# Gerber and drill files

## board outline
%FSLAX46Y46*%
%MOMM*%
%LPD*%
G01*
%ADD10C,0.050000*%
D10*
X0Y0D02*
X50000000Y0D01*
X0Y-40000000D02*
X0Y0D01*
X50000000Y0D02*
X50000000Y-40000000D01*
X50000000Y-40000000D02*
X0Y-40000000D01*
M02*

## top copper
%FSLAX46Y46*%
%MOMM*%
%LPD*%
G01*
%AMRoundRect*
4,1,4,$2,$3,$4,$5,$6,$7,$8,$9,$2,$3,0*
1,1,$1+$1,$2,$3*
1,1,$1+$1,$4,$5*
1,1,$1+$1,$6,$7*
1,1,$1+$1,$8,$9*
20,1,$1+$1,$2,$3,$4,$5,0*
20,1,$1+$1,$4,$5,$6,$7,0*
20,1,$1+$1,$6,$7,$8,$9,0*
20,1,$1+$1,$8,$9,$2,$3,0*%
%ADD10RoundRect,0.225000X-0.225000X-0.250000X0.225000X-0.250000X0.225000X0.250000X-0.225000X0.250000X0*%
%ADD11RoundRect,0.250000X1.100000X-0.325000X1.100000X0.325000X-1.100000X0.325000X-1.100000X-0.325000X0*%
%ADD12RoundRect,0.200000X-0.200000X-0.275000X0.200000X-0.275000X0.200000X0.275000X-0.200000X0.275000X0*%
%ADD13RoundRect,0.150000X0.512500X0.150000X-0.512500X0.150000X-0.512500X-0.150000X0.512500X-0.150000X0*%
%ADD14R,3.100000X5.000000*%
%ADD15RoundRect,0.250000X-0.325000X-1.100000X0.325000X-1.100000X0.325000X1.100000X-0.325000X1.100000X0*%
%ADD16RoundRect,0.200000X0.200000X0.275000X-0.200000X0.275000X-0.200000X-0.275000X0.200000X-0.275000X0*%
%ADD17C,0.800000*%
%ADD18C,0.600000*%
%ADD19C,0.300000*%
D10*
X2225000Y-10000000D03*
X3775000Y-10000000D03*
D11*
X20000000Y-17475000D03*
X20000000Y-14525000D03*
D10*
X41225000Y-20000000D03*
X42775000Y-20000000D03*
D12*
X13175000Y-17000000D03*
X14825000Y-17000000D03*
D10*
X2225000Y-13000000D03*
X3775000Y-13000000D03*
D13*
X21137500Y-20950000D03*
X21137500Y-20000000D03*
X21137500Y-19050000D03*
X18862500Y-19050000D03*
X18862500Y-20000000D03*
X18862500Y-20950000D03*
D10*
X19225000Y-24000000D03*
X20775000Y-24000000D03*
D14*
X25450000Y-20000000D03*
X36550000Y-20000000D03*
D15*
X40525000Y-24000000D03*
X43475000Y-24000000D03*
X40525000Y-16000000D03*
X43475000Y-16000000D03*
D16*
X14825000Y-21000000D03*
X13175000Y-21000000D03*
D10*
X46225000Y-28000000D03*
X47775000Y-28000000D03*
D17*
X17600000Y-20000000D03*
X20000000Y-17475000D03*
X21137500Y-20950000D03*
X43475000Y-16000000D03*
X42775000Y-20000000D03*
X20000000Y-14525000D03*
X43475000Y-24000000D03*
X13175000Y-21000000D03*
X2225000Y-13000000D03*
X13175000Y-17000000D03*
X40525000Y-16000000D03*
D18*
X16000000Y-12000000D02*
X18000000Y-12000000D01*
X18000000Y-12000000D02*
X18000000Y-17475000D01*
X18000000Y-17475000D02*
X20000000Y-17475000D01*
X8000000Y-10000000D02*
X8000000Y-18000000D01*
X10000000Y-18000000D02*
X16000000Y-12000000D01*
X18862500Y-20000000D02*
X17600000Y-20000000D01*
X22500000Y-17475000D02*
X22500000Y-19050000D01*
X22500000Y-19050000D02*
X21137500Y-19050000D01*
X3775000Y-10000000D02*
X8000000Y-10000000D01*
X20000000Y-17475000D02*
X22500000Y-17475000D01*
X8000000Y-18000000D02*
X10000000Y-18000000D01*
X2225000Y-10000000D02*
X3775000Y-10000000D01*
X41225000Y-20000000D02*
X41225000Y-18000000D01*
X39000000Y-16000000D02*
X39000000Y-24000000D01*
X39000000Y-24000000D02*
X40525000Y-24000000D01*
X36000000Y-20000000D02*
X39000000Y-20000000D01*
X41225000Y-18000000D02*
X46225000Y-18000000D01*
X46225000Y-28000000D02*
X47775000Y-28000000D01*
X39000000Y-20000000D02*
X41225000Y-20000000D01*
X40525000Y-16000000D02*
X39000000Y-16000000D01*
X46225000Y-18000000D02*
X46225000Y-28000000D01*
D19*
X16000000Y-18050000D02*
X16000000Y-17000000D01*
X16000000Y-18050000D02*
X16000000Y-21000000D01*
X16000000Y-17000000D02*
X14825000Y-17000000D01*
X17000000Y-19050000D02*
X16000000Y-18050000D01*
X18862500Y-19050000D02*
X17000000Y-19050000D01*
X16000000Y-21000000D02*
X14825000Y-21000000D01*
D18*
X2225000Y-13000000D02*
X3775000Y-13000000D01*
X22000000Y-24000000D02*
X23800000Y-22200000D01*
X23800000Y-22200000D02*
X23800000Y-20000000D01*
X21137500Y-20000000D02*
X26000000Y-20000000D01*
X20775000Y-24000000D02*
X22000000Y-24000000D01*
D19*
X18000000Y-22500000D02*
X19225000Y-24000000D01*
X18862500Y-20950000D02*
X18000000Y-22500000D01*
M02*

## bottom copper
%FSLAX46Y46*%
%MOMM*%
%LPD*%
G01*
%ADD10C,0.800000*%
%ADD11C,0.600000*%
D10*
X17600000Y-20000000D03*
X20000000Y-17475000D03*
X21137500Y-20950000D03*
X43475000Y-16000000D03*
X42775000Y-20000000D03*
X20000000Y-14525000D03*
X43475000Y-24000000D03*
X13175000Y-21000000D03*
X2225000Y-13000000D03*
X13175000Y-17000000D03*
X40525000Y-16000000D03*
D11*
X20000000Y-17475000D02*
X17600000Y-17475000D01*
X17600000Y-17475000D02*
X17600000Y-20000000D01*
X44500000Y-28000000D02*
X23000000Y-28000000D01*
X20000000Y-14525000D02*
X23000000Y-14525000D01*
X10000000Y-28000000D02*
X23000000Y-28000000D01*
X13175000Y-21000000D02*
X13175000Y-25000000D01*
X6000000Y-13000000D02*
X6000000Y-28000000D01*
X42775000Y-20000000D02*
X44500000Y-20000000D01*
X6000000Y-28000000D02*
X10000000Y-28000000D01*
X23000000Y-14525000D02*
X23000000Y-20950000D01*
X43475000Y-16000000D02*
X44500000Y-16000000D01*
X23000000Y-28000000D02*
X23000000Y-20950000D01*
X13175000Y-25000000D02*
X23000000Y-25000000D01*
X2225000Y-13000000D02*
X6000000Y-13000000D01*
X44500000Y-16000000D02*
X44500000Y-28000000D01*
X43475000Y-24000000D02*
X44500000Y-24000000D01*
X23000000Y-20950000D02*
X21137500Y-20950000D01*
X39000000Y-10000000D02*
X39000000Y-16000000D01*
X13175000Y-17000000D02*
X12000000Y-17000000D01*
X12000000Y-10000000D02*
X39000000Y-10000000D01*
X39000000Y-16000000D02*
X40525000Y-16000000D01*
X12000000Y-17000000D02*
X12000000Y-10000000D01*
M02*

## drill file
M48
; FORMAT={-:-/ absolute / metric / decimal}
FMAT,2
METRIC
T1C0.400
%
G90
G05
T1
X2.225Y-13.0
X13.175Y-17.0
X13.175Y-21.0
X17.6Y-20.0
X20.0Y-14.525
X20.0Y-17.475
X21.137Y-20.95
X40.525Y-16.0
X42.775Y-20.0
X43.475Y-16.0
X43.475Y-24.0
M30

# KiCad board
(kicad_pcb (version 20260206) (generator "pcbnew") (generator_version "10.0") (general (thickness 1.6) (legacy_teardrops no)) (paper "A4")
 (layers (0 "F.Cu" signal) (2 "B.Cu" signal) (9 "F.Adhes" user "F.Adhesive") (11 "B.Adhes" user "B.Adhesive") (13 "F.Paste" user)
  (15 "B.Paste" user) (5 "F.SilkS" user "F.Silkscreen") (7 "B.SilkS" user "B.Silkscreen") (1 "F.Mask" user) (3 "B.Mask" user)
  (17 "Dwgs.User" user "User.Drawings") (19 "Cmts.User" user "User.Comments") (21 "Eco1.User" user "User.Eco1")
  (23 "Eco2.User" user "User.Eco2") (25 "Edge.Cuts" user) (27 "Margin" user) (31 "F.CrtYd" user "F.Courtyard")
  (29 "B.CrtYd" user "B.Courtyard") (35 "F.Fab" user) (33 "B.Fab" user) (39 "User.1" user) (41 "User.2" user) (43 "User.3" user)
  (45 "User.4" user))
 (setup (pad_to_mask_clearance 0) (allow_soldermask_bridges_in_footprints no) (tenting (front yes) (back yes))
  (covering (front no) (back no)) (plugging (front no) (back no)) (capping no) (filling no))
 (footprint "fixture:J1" (layer "F.Cu") (at 3 10)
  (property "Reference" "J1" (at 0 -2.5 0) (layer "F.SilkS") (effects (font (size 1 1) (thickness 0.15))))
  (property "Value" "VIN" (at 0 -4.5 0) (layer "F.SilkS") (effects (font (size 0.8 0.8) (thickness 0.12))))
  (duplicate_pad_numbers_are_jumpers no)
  (pad "1" smd roundrect (at -0.775 0) (size 0.9 0.95) (layers "F.Cu" "F.Mask" "F.Paste") (roundrect_rratio 0.25) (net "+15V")
   (thermal_bridge_angle 45))
  (pad "2" smd roundrect (at 0.775 0) (size 0.9 0.95) (layers "F.Cu" "F.Mask" "F.Paste") (roundrect_rratio 0.25) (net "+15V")
   (thermal_bridge_angle 45)))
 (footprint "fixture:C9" (layer "F.Cu") (at 20 16 90)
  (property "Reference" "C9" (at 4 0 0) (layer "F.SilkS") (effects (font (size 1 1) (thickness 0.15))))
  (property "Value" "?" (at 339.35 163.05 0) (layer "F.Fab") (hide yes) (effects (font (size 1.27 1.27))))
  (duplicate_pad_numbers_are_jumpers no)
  (pad "1" smd roundrect (at -1.475 0 90) (size 1.15 2.7) (layers "F.Cu" "F.Mask" "F.Paste") (roundrect_rratio 0.217391) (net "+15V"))
  (pad "2" smd roundrect (at 1.475 0 90) (size 1.15 2.7) (layers "F.Cu" "F.Mask" "F.Paste") (roundrect_rratio 0.217391) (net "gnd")))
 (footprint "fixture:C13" (layer "F.Cu") (at 42 20)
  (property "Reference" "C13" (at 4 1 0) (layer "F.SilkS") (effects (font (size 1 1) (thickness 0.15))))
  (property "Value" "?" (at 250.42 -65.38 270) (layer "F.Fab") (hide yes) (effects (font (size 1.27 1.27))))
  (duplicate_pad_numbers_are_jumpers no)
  (pad "1" smd roundrect (at -0.775 0) (size 0.9 0.95) (layers "F.Cu" "F.Mask" "F.Paste") (roundrect_rratio 0.25) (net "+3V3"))
  (pad "2" smd roundrect (at 0.775 0) (size 0.9 0.95) (layers "F.Cu" "F.Mask" "F.Paste") (roundrect_rratio 0.25) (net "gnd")))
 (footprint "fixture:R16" (layer "F.Cu") (at 14 17)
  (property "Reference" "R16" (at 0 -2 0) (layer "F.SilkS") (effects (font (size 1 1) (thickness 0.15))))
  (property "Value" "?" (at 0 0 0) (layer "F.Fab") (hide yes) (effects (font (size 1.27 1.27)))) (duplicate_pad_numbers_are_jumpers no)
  (pad "1" smd roundrect (at -0.825 0) (size 0.8 0.95) (layers "F.Cu" "F.Mask" "F.Paste") (roundrect_rratio 0.25) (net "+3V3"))
  (pad "2" smd roundrect (at 0.825 0) (size 0.8 0.95) (layers "F.Cu" "F.Mask" "F.Paste") (roundrect_rratio 0.25) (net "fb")))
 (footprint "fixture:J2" (layer "F.Cu") (at 3 13)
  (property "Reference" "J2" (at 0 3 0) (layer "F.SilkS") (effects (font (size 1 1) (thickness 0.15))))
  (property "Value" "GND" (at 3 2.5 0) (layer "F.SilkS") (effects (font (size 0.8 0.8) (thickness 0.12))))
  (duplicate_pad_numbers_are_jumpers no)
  (pad "1" smd roundrect (at -0.775 0) (size 0.9 0.95) (layers "F.Cu" "F.Mask" "F.Paste") (roundrect_rratio 0.25) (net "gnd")
   (thermal_bridge_angle 45))
  (pad "2" smd roundrect (at 0.775 0) (size 0.9 0.95) (layers "F.Cu" "F.Mask" "F.Paste") (roundrect_rratio 0.25) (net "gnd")
   (thermal_bridge_angle 45)))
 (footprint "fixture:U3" (layer "F.Cu") (at 20 20 180)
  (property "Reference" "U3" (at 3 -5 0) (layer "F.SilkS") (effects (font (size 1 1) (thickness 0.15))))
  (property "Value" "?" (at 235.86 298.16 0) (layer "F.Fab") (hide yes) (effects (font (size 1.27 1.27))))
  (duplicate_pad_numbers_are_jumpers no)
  (pad "1" smd roundrect (at -1.1375 -0.95 180) (size 1.325 0.6) (layers "F.Cu" "F.Mask" "F.Paste") (roundrect_rratio 0.25) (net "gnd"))
  (pad "2" smd roundrect (at -1.1375 0 180) (size 1.325 0.6) (layers "F.Cu" "F.Mask" "F.Paste") (roundrect_rratio 0.25) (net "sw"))
  (pad "3" smd roundrect (at -1.1375 0.95 180) (size 1.325 0.6) (layers "F.Cu" "F.Mask" "F.Paste") (roundrect_rratio 0.25) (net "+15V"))
  (pad "4" smd roundrect (at 1.1375 0.95 180) (size 1.325 0.6) (layers "F.Cu" "F.Mask" "F.Paste") (roundrect_rratio 0.25) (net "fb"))
  (pad "5" smd roundrect (at 1.1375 0 180) (size 1.325 0.6) (layers "F.Cu" "F.Mask" "F.Paste") (roundrect_rratio 0.25) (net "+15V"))
  (pad "6" smd roundrect (at 1.1375 -0.95 180) (size 1.325 0.6) (layers "F.Cu" "F.Mask" "F.Paste") (roundrect_rratio 0.25) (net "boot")))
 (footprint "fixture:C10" (layer "F.Cu") (at 20 24)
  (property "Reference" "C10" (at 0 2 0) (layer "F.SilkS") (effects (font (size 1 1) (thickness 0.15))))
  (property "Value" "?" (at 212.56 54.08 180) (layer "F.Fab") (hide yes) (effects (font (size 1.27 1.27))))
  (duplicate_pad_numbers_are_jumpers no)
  (pad "1" smd roundrect (at -0.775 0) (size 0.9 0.95) (layers "F.Cu" "F.Mask" "F.Paste") (roundrect_rratio 0.25) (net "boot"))
  (pad "2" smd roundrect (at 0.775 0) (size 0.9 0.95) (layers "F.Cu" "F.Mask" "F.Paste") (roundrect_rratio 0.25) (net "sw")))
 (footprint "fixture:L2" (layer "F.Cu") (at 31 20)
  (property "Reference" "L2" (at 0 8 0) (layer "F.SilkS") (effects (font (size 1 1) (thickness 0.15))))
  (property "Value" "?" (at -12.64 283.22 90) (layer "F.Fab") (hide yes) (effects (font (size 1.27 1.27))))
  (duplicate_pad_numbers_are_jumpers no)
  (pad "1" smd rect (at -5.55 0) (size 3.1 5) (layers "F.Cu" "F.Mask" "F.Paste") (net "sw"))
  (pad "2" smd rect (at 5.55 0) (size 3.1 5) (layers "F.Cu" "F.Mask" "F.Paste") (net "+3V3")))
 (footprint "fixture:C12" (layer "F.Cu") (at 42 24)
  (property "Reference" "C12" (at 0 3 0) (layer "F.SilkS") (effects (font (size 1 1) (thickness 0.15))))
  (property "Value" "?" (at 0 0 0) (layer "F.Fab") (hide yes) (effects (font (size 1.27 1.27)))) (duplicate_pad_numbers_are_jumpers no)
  (pad "1" smd roundrect (at -1.475 0) (size 1.15 2.7) (layers "F.Cu" "F.Mask" "F.Paste") (roundrect_rratio 0.217391) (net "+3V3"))
  (pad "2" smd roundrect (at 1.475 0) (size 1.15 2.7) (layers "F.Cu" "F.Mask" "F.Paste") (roundrect_rratio 0.217391) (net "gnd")))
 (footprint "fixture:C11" (layer "F.Cu") (at 42 16)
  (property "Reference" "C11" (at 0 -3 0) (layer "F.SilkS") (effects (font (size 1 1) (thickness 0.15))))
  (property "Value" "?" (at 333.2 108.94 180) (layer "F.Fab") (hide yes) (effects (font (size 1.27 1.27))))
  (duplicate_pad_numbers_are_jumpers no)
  (pad "1" smd roundrect (at -1.475 0) (size 1.15 2.7) (layers "F.Cu" "F.Mask" "F.Paste") (roundrect_rratio 0.217391) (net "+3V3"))
  (pad "2" smd roundrect (at 1.475 0) (size 1.15 2.7) (layers "F.Cu" "F.Mask" "F.Paste") (roundrect_rratio 0.217391) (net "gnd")))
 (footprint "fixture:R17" (layer "F.Cu") (at 14 21 180)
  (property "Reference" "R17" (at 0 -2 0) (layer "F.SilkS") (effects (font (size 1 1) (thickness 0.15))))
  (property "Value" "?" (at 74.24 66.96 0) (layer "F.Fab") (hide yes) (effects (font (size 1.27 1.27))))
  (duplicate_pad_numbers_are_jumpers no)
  (pad "1" smd roundrect (at -0.825 0 180) (size 0.8 0.95) (layers "F.Cu" "F.Mask" "F.Paste") (roundrect_rratio 0.25) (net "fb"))
  (pad "2" smd roundrect (at 0.825 0 180) (size 0.8 0.95) (layers "F.Cu" "F.Mask" "F.Paste") (roundrect_rratio 0.25) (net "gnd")))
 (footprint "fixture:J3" (layer "F.Cu") (at 47 28)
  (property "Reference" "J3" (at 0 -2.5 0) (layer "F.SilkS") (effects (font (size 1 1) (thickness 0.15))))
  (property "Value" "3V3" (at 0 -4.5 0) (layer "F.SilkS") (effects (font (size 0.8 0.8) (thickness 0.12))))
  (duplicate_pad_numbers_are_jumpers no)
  (pad "1" smd roundrect (at -0.775 0) (size 0.9 0.95) (layers "F.Cu" "F.Mask" "F.Paste") (roundrect_rratio 0.25) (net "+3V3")
   (thermal_bridge_angle 45))
  (pad "2" smd roundrect (at 0.775 0) (size 0.9 0.95) (layers "F.Cu" "F.Mask" "F.Paste") (roundrect_rratio 0.25) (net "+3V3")
   (thermal_bridge_angle 45)))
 (gr_line (start 0 0) (end 50 0) (stroke (width 0.05) (type default)) (layer "Edge.Cuts"))
 (gr_line (start 0 40) (end 0 0) (stroke (width 0.05) (type default)) (layer "Edge.Cuts"))
 (gr_line (start 50 0) (end 50 40) (stroke (width 0.05) (type default)) (layer "Edge.Cuts"))
 (gr_line (start 50 40) (end 0 40) (stroke (width 0.05) (type default)) (layer "Edge.Cuts"))
 (segment (start 16 12) (end 18 12) (width 0.6) (layer "F.Cu") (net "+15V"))
 (segment (start 18 12) (end 18 17.475) (width 0.6) (layer "F.Cu") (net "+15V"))
 (segment (start 18 17.475) (end 20 17.475) (width 0.6) (layer "F.Cu") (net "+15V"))
 (segment (start 8 10) (end 8 18) (width 0.6) (layer "F.Cu") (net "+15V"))
 (segment (start 10 18) (end 16 12) (width 0.6) (layer "F.Cu") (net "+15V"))
 (segment (start 18.8625 20) (end 17.6 20) (width 0.6) (layer "F.Cu") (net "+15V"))
 (segment (start 22.5 17.475) (end 22.5 19.05) (width 0.6) (layer "F.Cu") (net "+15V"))
 (segment (start 22.5 19.05) (end 21.1375 19.05) (width 0.6) (layer "F.Cu") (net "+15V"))
 (segment (start 3.775 10) (end 8 10) (width 0.6) (layer "F.Cu") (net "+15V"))
 (segment (start 20 17.475) (end 22.5 17.475) (width 0.6) (layer "F.Cu") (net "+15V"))
 (segment (start 8 18) (end 10 18) (width 0.6) (layer "F.Cu") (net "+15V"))
 (segment (start 2.225 10) (end 3.775 10) (width 0.6) (layer "F.Cu") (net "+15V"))
 (via (at 17.6 20) (size 0.8) (drill 0.4) (layers "F.Cu" "B.Cu") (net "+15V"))
 (via (at 20 17.475) (size 0.8) (drill 0.4) (layers "F.Cu" "B.Cu") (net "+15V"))
 (segment (start 20 17.475) (end 17.6 17.475) (width 0.6) (layer "B.Cu") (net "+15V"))
 (segment (start 17.6 17.475) (end 17.6 20) (width 0.6) (layer "B.Cu") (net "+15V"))
 (via (at 21.1375 20.95) (size 0.8) (drill 0.4) (layers "F.Cu" "B.Cu") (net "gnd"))
 (via (at 43.475 16) (size 0.8) (drill 0.4) (layers "F.Cu" "B.Cu") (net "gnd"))
 (via (at 42.775 20) (size 0.8) (drill 0.4) (layers "F.Cu" "B.Cu") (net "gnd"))
 (via (at 20 14.525) (size 0.8) (drill 0.4) (layers "F.Cu" "B.Cu") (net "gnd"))
 (via (at 43.475 24) (size 0.8) (drill 0.4) (layers "F.Cu" "B.Cu") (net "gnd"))
 (via (at 13.175 21) (size 0.8) (drill 0.4) (layers "F.Cu" "B.Cu") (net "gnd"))
 (via (at 2.225 13) (size 0.8) (drill 0.4) (layers "F.Cu" "B.Cu") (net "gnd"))
 (segment (start 44.5 28) (end 23 28) (width 0.6) (layer "B.Cu") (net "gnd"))
 (segment (start 20 14.525) (end 23 14.525) (width 0.6) (layer "B.Cu") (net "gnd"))
 (segment (start 10 28) (end 23 28) (width 0.6) (layer "B.Cu") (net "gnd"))
 (segment (start 13.175 21) (end 13.175 25) (width 0.6) (layer "B.Cu") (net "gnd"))
 (segment (start 6 13) (end 6 28) (width 0.6) (layer "B.Cu") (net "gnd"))
 (segment (start 42.775 20) (end 44.5 20) (width 0.6) (layer "B.Cu") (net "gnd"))
 (segment (start 6 28) (end 10 28) (width 0.6) (layer "B.Cu") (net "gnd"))
 (segment (start 23 14.525) (end 23 20.95) (width 0.6) (layer "B.Cu") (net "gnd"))
 (segment (start 43.475 16) (end 44.5 16) (width 0.6) (layer "B.Cu") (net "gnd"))
 (segment (start 23 28) (end 23 20.95) (width 0.6) (layer "B.Cu") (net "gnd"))
 (segment (start 13.175 25) (end 23 25) (width 0.6) (layer "B.Cu") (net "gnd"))
 (segment (start 2.225 13) (end 6 13) (width 0.6) (layer "B.Cu") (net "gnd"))
 (segment (start 44.5 16) (end 44.5 28) (width 0.6) (layer "B.Cu") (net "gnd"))
 (segment (start 43.475 24) (end 44.5 24) (width 0.6) (layer "B.Cu") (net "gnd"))
 (segment (start 23 20.95) (end 21.1375 20.95) (width 0.6) (layer "B.Cu") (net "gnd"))
 (segment (start 41.225 20) (end 41.225 18) (width 0.6) (layer "F.Cu") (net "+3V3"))
 (segment (start 39 16) (end 39 24) (width 0.6) (layer "F.Cu") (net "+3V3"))
 (segment (start 39 24) (end 40.525 24) (width 0.6) (layer "F.Cu") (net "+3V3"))
 (segment (start 36 20) (end 39 20) (width 0.6) (layer "F.Cu") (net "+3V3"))
 (segment (start 41.225 18) (end 46.225 18) (width 0.6) (layer "F.Cu") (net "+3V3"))
 (segment (start 46.225 28) (end 47.775 28) (width 0.6) (layer "F.Cu") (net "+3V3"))
 (segment (start 39 20) (end 41.225 20) (width 0.6) (layer "F.Cu") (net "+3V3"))
 (segment (start 40.525 16) (end 39 16) (width 0.6) (layer "F.Cu") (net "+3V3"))
 (segment (start 46.225 18) (end 46.225 28) (width 0.6) (layer "F.Cu") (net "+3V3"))
 (via (at 13.175 17) (size 0.8) (drill 0.4) (layers "F.Cu" "B.Cu") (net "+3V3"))
 (via (at 40.525 16) (size 0.8) (drill 0.4) (layers "F.Cu" "B.Cu") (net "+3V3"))
 (segment (start 39 10) (end 39 16) (width 0.6) (layer "B.Cu") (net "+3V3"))
 (segment (start 13.175 17) (end 12 17) (width 0.6) (layer "B.Cu") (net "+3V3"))
 (segment (start 12 10) (end 39 10) (width 0.6) (layer "B.Cu") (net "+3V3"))
 (segment (start 39 16) (end 40.525 16) (width 0.6) (layer "B.Cu") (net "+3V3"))
 (segment (start 12 17) (end 12 10) (width 0.6) (layer "B.Cu") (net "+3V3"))
 (segment (start 16 18.05) (end 16 17) (width 0.3) (layer "F.Cu") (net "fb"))
 (segment (start 16 18.05) (end 16 21) (width 0.3) (layer "F.Cu") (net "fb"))
 (segment (start 16 17) (end 14.825 17) (width 0.3) (layer "F.Cu") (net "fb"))
 (segment (start 17 19.05) (end 16 18.05) (width 0.3) (layer "F.Cu") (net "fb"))
 (segment (start 18.8625 19.05) (end 17 19.05) (width 0.3) (layer "F.Cu") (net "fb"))
 (segment (start 16 21) (end 14.825 21) (width 0.3) (layer "F.Cu") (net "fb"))
 (segment (start 2.225 13) (end 3.775 13) (width 0.6) (layer "F.Cu") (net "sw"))
 (segment (start 22 24) (end 23.8 22.2) (width 0.6) (layer "F.Cu") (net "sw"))
 (segment (start 23.8 22.2) (end 23.8 20) (width 0.6) (layer "F.Cu") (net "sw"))
 (segment (start 21.1375 20) (end 26 20) (width 0.6) (layer "F.Cu") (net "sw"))
 (segment (start 20.775 24) (end 22 24) (width 0.6) (layer "F.Cu") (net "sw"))
 (segment (start 18 22.5) (end 19.225 24) (width 0.3) (layer "F.Cu") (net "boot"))
 (segment (start 18.8625 20.95) (end 18 22.5) (width 0.3) (layer "F.Cu") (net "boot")))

